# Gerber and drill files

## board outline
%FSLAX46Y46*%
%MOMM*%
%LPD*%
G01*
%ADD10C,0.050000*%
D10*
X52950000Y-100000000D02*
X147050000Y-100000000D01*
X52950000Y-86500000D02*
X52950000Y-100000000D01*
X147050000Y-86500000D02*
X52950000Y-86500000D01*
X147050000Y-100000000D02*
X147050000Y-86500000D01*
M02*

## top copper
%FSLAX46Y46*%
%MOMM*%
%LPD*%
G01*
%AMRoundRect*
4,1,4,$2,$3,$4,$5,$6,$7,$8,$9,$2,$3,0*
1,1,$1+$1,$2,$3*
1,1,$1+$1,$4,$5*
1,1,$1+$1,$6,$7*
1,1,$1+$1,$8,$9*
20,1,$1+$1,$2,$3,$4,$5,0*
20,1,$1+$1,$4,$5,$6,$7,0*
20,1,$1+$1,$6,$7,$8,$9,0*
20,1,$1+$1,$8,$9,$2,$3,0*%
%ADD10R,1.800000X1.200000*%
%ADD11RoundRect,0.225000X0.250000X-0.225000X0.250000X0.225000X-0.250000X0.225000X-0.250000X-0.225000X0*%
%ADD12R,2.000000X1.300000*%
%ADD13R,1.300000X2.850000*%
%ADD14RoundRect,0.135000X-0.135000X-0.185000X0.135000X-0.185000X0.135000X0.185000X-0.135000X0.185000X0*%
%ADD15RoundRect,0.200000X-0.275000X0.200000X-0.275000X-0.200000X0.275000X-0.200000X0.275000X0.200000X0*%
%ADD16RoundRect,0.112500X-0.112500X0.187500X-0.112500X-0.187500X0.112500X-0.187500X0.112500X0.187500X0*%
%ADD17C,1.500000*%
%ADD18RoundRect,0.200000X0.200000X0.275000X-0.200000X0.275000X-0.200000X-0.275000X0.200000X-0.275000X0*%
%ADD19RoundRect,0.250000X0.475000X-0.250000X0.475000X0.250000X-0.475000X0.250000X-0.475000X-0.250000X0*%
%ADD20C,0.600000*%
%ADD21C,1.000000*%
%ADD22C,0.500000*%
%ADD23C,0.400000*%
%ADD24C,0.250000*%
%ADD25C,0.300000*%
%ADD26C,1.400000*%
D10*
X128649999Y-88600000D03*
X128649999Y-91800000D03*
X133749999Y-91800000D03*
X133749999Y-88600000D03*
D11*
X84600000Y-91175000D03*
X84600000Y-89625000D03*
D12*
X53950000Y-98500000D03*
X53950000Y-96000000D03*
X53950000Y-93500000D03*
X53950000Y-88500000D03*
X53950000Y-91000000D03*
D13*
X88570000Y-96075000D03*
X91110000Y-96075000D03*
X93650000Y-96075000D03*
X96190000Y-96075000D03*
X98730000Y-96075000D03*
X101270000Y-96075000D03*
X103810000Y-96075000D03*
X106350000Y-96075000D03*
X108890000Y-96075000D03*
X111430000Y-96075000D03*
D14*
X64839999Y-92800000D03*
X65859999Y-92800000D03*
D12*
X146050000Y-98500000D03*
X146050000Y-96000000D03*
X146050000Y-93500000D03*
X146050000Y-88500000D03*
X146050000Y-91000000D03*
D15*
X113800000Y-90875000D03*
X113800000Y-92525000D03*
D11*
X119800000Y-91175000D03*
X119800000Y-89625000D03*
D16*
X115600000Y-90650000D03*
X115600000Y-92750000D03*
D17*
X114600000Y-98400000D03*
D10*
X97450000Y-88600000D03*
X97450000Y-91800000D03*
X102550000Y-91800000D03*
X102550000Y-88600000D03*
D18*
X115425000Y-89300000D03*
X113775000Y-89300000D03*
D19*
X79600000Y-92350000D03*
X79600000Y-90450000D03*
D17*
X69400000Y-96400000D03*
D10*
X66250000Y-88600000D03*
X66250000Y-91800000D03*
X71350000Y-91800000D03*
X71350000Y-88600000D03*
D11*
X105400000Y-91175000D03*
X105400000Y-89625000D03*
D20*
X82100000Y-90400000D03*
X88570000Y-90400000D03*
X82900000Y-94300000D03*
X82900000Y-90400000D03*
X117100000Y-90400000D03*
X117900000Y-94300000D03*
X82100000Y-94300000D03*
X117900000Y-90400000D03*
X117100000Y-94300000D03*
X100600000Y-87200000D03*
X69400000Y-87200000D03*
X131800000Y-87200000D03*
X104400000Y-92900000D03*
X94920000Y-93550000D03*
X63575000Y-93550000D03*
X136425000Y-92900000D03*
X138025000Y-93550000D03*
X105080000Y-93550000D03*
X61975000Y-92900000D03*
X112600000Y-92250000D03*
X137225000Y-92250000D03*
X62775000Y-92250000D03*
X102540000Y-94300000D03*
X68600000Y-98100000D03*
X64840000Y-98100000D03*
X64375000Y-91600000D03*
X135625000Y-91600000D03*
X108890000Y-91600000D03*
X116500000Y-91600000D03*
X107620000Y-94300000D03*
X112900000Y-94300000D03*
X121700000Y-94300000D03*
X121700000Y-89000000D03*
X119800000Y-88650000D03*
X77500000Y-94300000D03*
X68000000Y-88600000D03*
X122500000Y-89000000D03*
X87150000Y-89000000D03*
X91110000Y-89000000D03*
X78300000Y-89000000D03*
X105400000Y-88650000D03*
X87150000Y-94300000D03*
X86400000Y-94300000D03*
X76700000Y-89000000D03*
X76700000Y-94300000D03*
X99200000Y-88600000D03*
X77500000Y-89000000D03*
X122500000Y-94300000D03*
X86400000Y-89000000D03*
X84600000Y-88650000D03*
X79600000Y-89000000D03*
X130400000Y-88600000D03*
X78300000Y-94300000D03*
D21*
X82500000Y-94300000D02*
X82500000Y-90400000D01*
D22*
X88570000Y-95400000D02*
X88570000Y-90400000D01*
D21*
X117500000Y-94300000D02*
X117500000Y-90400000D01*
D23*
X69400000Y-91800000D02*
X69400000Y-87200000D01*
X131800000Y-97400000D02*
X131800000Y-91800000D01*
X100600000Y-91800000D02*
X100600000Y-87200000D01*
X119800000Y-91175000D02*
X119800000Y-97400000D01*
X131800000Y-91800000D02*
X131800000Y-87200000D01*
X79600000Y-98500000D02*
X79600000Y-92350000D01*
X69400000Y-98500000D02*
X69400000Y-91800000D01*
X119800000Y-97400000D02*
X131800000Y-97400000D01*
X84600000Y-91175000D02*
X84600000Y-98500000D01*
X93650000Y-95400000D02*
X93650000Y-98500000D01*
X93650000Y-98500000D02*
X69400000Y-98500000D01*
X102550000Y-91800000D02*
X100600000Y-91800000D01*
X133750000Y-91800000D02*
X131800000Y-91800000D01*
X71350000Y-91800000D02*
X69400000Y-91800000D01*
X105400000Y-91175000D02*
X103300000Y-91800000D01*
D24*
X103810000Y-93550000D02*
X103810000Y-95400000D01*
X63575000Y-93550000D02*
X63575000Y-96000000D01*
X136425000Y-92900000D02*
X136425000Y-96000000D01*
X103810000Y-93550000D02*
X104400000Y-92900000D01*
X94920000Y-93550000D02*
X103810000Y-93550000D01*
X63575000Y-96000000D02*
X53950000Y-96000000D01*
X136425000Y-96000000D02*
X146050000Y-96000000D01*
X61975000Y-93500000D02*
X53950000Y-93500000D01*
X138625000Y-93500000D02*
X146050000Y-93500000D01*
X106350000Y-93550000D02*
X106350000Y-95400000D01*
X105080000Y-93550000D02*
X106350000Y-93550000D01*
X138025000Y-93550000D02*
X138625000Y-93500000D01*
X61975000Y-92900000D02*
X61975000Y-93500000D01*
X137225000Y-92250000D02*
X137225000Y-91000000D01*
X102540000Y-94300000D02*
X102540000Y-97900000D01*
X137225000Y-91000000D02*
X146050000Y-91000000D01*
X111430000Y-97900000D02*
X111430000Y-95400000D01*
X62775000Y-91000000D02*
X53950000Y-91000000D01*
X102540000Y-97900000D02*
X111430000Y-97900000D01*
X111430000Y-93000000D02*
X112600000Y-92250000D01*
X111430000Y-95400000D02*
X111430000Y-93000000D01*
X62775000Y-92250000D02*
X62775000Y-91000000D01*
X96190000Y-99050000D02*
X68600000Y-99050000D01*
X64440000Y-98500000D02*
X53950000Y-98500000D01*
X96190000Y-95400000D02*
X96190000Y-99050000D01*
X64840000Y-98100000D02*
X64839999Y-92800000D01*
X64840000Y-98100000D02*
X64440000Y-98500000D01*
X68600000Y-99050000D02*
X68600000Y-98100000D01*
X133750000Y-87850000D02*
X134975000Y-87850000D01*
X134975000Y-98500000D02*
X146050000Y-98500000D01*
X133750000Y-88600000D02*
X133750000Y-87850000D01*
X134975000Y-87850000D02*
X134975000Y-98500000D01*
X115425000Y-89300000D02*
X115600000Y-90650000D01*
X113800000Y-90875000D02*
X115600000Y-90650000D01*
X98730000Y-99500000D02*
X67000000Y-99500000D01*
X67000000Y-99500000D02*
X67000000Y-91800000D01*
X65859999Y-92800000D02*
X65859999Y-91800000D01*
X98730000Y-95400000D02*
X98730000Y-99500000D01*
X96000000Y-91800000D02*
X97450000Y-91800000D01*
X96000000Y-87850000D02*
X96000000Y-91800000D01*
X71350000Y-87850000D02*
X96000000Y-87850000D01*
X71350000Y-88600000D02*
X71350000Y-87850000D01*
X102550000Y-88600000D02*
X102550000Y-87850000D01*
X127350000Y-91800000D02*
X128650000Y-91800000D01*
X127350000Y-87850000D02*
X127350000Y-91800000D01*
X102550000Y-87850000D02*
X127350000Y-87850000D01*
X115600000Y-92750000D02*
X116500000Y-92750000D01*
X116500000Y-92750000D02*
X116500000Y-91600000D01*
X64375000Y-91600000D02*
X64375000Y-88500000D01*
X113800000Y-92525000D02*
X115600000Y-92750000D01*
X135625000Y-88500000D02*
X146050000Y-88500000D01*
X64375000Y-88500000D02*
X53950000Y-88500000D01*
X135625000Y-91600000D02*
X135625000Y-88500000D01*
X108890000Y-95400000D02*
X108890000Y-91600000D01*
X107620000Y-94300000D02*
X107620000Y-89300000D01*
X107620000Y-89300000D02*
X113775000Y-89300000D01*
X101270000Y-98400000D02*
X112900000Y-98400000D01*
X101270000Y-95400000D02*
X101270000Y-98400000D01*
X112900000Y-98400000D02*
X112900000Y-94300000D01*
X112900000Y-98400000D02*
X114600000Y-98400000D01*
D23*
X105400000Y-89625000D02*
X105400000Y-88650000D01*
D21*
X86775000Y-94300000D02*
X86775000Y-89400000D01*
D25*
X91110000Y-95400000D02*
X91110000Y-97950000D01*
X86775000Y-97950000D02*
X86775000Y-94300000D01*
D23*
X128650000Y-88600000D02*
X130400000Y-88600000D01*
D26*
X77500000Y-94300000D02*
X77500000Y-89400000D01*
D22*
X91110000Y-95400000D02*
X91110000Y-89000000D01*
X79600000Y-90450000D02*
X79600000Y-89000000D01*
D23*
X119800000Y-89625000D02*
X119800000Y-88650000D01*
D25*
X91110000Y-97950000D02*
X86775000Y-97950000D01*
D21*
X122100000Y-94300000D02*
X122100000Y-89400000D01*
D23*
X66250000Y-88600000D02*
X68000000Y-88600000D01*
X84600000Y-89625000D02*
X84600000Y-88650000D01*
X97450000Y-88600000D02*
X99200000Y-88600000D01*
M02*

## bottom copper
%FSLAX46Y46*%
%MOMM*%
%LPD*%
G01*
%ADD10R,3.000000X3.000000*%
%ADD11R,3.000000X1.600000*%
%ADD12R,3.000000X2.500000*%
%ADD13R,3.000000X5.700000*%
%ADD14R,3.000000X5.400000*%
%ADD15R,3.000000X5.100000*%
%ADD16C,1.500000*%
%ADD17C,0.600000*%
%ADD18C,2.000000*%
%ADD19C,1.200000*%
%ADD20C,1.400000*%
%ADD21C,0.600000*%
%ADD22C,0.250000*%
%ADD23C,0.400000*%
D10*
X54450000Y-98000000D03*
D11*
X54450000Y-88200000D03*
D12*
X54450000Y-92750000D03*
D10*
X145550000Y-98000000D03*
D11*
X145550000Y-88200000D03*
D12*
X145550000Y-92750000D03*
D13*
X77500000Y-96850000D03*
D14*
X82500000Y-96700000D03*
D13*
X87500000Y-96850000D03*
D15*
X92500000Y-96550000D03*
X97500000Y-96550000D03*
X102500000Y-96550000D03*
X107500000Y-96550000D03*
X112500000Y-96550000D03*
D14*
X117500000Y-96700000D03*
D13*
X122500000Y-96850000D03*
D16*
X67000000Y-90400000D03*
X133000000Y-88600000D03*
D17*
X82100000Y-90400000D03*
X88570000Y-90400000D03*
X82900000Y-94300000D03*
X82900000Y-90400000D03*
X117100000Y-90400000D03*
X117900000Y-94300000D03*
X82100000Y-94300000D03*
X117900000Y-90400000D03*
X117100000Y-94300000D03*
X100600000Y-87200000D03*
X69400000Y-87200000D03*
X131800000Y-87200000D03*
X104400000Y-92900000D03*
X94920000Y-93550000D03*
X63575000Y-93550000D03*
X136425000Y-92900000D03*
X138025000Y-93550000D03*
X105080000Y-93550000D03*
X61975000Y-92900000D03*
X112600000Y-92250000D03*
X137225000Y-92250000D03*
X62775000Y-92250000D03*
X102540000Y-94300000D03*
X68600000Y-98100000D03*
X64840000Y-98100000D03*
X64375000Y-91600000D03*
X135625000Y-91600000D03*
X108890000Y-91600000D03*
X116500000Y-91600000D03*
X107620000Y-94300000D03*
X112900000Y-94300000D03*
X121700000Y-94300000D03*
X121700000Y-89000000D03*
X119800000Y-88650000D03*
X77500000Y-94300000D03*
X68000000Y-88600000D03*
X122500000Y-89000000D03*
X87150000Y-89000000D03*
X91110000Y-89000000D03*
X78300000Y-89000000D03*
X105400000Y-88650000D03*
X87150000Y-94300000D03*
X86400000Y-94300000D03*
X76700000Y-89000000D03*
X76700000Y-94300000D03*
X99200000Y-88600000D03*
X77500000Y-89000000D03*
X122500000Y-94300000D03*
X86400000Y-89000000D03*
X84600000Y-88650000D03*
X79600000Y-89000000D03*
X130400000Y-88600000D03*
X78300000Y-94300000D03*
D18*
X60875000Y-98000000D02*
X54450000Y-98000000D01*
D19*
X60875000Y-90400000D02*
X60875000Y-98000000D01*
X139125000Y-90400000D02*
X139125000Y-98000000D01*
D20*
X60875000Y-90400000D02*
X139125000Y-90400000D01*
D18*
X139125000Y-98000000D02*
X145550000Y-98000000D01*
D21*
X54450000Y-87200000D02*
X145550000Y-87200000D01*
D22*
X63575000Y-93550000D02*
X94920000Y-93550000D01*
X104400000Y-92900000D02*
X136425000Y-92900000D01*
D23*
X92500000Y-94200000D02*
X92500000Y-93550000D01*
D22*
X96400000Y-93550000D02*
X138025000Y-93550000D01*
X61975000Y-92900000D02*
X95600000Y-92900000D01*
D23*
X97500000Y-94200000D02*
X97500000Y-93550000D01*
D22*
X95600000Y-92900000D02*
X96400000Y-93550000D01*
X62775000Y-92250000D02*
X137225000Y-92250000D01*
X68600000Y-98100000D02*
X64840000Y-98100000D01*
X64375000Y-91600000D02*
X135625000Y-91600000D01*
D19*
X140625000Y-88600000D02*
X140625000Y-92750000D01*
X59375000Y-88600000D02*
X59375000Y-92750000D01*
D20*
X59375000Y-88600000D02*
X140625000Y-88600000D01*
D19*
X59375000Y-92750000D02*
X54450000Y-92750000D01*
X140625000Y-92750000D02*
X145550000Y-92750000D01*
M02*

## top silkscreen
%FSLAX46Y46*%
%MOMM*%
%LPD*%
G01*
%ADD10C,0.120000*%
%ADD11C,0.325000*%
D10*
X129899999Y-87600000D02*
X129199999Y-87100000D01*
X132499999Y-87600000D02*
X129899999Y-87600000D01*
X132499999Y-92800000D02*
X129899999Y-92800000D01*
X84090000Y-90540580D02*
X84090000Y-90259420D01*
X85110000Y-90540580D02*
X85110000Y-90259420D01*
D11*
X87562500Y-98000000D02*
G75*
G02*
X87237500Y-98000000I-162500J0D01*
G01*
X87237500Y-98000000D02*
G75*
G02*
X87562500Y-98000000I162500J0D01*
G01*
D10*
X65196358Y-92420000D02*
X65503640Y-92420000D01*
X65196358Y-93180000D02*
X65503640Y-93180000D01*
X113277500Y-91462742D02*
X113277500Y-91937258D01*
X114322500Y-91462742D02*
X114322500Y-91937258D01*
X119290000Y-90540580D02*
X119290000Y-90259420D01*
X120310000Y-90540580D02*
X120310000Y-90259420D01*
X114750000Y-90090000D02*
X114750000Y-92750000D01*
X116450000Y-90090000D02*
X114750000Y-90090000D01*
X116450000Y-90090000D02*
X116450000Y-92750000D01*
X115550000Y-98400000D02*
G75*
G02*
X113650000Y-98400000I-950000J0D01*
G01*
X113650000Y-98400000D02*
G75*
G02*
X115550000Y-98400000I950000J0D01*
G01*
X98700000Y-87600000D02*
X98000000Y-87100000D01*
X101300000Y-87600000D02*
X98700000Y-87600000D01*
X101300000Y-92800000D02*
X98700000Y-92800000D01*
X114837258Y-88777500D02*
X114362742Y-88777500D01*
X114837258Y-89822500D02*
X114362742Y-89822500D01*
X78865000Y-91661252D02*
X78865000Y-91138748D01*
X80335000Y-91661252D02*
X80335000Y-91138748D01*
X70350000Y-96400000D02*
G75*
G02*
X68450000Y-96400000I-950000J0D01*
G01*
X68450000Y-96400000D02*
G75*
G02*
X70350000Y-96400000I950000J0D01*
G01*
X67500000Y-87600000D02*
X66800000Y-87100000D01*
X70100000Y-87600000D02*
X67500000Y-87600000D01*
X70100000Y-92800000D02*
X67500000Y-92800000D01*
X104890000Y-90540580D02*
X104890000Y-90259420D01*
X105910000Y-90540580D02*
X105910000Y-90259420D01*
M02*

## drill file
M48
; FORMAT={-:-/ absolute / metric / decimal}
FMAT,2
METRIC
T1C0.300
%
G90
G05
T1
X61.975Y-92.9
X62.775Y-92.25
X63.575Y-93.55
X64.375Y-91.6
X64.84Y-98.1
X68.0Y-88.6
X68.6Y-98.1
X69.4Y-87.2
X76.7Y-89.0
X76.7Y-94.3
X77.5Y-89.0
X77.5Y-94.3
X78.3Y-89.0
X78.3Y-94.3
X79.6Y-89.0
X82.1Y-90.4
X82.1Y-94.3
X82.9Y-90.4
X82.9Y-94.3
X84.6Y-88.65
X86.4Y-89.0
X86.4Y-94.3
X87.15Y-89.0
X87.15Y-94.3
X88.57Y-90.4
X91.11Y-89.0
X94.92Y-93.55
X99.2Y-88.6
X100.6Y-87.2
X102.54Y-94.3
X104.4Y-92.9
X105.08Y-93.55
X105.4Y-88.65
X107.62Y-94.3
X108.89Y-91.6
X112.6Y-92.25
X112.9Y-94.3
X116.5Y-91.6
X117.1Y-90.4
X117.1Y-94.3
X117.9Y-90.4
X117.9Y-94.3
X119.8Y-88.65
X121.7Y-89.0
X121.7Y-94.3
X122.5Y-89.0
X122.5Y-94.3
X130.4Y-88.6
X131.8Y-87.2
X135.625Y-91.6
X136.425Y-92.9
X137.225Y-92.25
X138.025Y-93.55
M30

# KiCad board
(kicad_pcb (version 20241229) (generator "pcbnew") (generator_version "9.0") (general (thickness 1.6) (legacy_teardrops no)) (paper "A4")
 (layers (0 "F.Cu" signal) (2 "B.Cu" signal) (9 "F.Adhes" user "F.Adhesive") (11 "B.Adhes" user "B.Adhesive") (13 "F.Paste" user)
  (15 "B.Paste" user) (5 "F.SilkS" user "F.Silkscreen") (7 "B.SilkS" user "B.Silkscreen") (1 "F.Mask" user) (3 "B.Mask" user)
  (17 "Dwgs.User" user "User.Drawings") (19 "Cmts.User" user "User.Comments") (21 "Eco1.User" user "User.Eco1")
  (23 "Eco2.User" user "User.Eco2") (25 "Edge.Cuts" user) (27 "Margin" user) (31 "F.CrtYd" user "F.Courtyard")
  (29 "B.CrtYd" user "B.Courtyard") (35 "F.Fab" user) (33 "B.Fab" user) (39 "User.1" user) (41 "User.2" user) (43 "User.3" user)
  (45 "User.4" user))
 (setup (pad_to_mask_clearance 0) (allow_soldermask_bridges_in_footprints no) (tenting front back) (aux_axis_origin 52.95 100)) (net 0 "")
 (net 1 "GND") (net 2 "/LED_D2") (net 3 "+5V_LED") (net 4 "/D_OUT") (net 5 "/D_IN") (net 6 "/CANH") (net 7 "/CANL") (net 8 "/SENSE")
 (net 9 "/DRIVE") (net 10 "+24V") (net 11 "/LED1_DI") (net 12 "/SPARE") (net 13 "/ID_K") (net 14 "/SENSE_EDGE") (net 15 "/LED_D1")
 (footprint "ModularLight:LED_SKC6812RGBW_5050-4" (layer "F.Cu") (at 131.199999 90.2 180)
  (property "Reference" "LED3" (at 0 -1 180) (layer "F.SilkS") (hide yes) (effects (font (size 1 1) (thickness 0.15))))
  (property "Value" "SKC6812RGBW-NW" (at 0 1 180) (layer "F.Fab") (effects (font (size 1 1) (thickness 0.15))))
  (fp_line (start 1.3 2.6) (end 2 3.1) (stroke (width 0.12) (type solid)) (layer "F.SilkS"))
  (fp_line (start -1.3 2.6) (end 1.3 2.6) (stroke (width 0.12) (type solid)) (layer "F.SilkS"))
  (fp_line (start -1.3 -2.6) (end 1.3 -2.6) (stroke (width 0.12) (type solid)) (layer "F.SilkS"))
  (pad "1" smd rect (at 2.55 1.6 180) (size 1.8 1.2) (layers "F.Cu" "F.Mask" "F.Paste") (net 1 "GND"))
  (pad "2" smd rect (at 2.55 -1.6 180) (size 1.8 1.2) (layers "F.Cu" "F.Mask" "F.Paste") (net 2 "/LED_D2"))
  (pad "3" smd rect (at -2.55 -1.6 180) (size 1.8 1.2) (layers "F.Cu" "F.Mask" "F.Paste") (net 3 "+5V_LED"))
  (pad "4" smd rect (at -2.55 1.6 180) (size 1.8 1.2) (layers "F.Cu" "F.Mask" "F.Paste") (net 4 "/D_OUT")))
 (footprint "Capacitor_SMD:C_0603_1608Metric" (layer "F.Cu") (at 84.6 90.4 90)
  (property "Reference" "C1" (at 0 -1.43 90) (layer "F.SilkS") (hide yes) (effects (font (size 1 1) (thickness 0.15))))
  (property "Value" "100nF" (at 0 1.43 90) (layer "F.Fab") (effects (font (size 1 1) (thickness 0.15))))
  (fp_line (start -0.14058 -0.51) (end 0.14058 -0.51) (stroke (width 0.12) (type solid)) (layer "F.SilkS"))
  (fp_line (start -0.14058 0.51) (end 0.14058 0.51) (stroke (width 0.12) (type solid)) (layer "F.SilkS"))
  (pad "1" smd roundrect (at -0.775 0 90) (size 0.9 0.95) (layers "F.Cu" "F.Mask" "F.Paste") (roundrect_rratio 0.25) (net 3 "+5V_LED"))
  (pad "2" smd roundrect (at 0.775 0 90) (size 0.9 0.95) (layers "F.Cu" "F.Mask" "F.Paste") (roundrect_rratio 0.25) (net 1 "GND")))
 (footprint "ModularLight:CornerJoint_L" (layer "F.Cu") (at 52.95 100)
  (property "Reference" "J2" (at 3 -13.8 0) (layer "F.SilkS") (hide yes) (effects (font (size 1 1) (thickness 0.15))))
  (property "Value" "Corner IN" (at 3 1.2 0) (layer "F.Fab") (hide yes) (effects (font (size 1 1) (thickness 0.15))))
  (pad "1" smd rect (at 1 -1.5) (size 2 1.3) (layers "F.Cu" "F.Mask" "F.Paste") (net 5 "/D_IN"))
  (pad "2" smd rect (at 1 -4) (size 2 1.3) (layers "F.Cu" "F.Mask" "F.Paste") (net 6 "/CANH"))
  (pad "3" smd rect (at 1 -6.5) (size 2 1.3) (layers "F.Cu" "F.Mask" "F.Paste") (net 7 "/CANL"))
  (pad "4" smd rect (at 1 -11.5) (size 2 1.3) (layers "F.Cu" "F.Mask" "F.Paste") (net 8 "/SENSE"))
  (pad "5" smd rect (at 1 -9) (size 2 1.3) (layers "F.Cu" "F.Mask" "F.Paste") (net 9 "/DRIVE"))
  (pad "6" smd rect (at 1.5 -2) (size 3 3) (layers "B.Cu" "B.Mask") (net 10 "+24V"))
  (pad "7" smd rect (at 1.5 -11.8) (size 3 1.6) (layers "B.Cu" "B.Mask") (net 3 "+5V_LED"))
  (pad "8" smd rect (at 1.5 -7.25) (size 3 2.5) (layers "B.Cu" "B.Mask") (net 1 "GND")))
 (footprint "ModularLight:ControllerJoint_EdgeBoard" (layer "F.Cu") (at 100 94.75)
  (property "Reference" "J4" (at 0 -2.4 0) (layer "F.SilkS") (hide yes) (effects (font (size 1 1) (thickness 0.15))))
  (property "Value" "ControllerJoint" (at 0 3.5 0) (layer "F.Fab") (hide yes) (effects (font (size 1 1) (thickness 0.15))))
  (fp_circle (center -12.6 3.25) (end -12.35 3.25) (stroke (width 0.15) (type solid)) (fill yes) (layer "F.SilkS"))
  (pad "1" smd rect (at -11.43 1.325) (size 1.3 2.85) (layers "F.Cu" "F.Mask" "F.Paste") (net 10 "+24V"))
  (pad "2" smd rect (at -8.89 1.325) (size 1.3 2.85) (layers "F.Cu" "F.Mask" "F.Paste") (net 1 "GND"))
  (pad "3" smd rect (at -6.35 1.325) (size 1.3 2.85) (layers "F.Cu" "F.Mask" "F.Paste") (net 3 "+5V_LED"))
  (pad "4" smd rect (at -3.81 1.325) (size 1.3 2.85) (layers "F.Cu" "F.Mask" "F.Paste") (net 5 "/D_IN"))
  (pad "5" smd rect (at -1.27 1.325) (size 1.3 2.85) (layers "F.Cu" "F.Mask" "F.Paste") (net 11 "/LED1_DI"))
  (pad "6" smd rect (at 1.27 1.325) (size 1.3 2.85) (layers "F.Cu" "F.Mask" "F.Paste") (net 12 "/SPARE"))
  (pad "7" smd rect (at 3.81 1.325) (size 1.3 2.85) (layers "F.Cu" "F.Mask" "F.Paste") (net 6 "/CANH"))
  (pad "8" smd rect (at 6.35 1.325) (size 1.3 2.85) (layers "F.Cu" "F.Mask" "F.Paste") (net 7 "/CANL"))
  (pad "9" smd rect (at 8.89 1.325) (size 1.3 2.85) (layers "F.Cu" "F.Mask" "F.Paste") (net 8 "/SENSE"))
  (pad "10" smd rect (at 11.43 1.325) (size 1.3 2.85) (layers "F.Cu" "F.Mask" "F.Paste") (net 9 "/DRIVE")))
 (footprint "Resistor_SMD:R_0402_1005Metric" (layer "F.Cu") (at 65.349999 92.8)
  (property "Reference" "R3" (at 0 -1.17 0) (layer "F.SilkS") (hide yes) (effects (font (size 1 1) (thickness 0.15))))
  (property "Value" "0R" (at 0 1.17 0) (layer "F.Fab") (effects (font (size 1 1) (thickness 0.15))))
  (fp_line (start -0.153641 -0.38) (end 0.153641 -0.38) (stroke (width 0.12) (type solid)) (layer "F.SilkS"))
  (fp_line (start -0.153641 0.38) (end 0.153641 0.38) (stroke (width 0.12) (type solid)) (layer "F.SilkS"))
  (pad "1" smd roundrect (at -0.51 0) (size 0.54 0.64) (layers "F.Cu" "F.Mask" "F.Paste") (roundrect_rratio 0.25) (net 5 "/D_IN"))
  (pad "2" smd roundrect (at 0.51 0) (size 0.54 0.64) (layers "F.Cu" "F.Mask" "F.Paste") (roundrect_rratio 0.25) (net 11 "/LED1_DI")))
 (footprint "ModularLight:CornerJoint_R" (layer "F.Cu") (at 147.05 100)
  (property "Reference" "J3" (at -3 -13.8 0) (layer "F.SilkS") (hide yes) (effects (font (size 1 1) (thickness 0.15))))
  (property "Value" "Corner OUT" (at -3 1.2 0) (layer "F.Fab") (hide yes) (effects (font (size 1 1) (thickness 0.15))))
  (pad "1" smd rect (at -1 -1.5) (size 2 1.3) (layers "F.Cu" "F.Mask" "F.Paste") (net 4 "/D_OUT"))
  (pad "2" smd rect (at -1 -4) (size 2 1.3) (layers "F.Cu" "F.Mask" "F.Paste") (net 6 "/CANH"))
  (pad "3" smd rect (at -1 -6.5) (size 2 1.3) (layers "F.Cu" "F.Mask" "F.Paste") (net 7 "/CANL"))
  (pad "4" smd rect (at -1 -11.5) (size 2 1.3) (layers "F.Cu" "F.Mask" "F.Paste") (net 8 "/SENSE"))
  (pad "5" smd rect (at -1 -9) (size 2 1.3) (layers "F.Cu" "F.Mask" "F.Paste") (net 9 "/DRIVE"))
  (pad "6" smd rect (at -1.5 -2) (size 3 3) (layers "B.Cu" "B.Mask") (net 10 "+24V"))
  (pad "7" smd rect (at -1.5 -11.8) (size 3 1.6) (layers "B.Cu" "B.Mask") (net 3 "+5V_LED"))
  (pad "8" smd rect (at -1.5 -7.25) (size 3 2.5) (layers "B.Cu" "B.Mask") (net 1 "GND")))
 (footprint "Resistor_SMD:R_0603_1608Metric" (layer "F.Cu") (at 113.8 91.7 -90)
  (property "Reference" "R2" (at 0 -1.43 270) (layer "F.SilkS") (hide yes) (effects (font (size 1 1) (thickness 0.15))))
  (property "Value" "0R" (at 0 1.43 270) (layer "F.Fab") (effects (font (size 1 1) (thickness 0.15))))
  (fp_line (start -0.237258 0.5225) (end 0.237258 0.5225) (stroke (width 0.12) (type solid)) (layer "F.SilkS"))
  (fp_line (start -0.237258 -0.5225) (end 0.237258 -0.5225) (stroke (width 0.12) (type solid)) (layer "F.SilkS"))
  (pad "1" smd roundrect (at -0.825 0 270) (size 0.8 0.95) (layers "F.Cu" "F.Mask" "F.Paste") (roundrect_rratio 0.25) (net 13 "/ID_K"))
  (pad "2" smd roundrect (at 0.825 0 270) (size 0.8 0.95) (layers "F.Cu" "F.Mask" "F.Paste") (roundrect_rratio 0.25) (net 8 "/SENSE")))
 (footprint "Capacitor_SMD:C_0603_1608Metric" (layer "F.Cu") (at 119.8 90.4 90)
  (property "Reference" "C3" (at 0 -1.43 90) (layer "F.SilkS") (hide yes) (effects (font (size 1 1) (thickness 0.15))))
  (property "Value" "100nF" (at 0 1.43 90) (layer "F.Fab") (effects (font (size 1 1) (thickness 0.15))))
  (fp_line (start -0.14058 -0.51) (end 0.14058 -0.51) (stroke (width 0.12) (type solid)) (layer "F.SilkS"))
  (fp_line (start -0.14058 0.51) (end 0.14058 0.51) (stroke (width 0.12) (type solid)) (layer "F.SilkS"))
  (pad "1" smd roundrect (at -0.775 0 90) (size 0.9 0.95) (layers "F.Cu" "F.Mask" "F.Paste") (roundrect_rratio 0.25) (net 3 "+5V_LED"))
  (pad "2" smd roundrect (at 0.775 0 90) (size 0.9 0.95) (layers "F.Cu" "F.Mask" "F.Paste") (roundrect_rratio 0.25) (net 1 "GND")))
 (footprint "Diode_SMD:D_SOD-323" (layer "F.Cu") (at 115.6 91.7 -90)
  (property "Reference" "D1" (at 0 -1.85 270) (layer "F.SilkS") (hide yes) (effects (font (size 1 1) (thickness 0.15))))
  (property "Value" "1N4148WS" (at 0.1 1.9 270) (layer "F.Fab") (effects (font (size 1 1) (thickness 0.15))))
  (fp_line (start -1.61 0.85) (end 1.05 0.85) (stroke (width 0.12) (type solid)) (layer "F.SilkS"))
  (fp_line (start -1.61 -0.85) (end -1.61 0.85) (stroke (width 0.12) (type solid)) (layer "F.SilkS"))
  (fp_line (start -1.61 -0.85) (end 1.05 -0.85) (stroke (width 0.12) (type solid)) (layer "F.SilkS"))
  (pad "1" smd roundrect (at -1.05 0 270) (size 0.6 0.45) (layers "F.Cu" "F.Mask" "F.Paste") (roundrect_rratio 0.25) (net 13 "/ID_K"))
  (pad "2" smd roundrect (at 1.05 0 270) (size 0.6 0.45) (layers "F.Cu" "F.Mask" "F.Paste") (roundrect_rratio 0.25) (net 8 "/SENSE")))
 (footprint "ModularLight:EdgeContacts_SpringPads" (layer "F.Cu") (at 100 100)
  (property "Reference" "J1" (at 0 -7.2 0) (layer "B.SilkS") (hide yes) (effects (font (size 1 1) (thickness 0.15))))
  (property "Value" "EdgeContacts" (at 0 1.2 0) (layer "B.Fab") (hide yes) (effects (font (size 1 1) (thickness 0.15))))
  (pad "X1" smd rect (at -22.5 -3.15) (size 3 5.7) (layers "B.Cu" "B.Mask") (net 1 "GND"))
  (pad "X2" smd rect (at -17.5 -3.3) (size 3 5.4) (layers "B.Cu" "B.Mask") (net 10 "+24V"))
  (pad "X3" smd rect (at -12.5 -3.15) (size 3 5.7) (layers "B.Cu" "B.Mask") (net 1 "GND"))
  (pad "X4" smd rect (at -7.5 -3.45) (size 3 5.1) (layers "B.Cu" "B.Mask") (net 6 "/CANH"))
  (pad "X5" smd rect (at -2.5 -3.45) (size 3 5.1) (layers "B.Cu" "B.Mask") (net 7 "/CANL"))
  (pad "X6" smd rect (at 2.5 -3.45) (size 3 5.1) (layers "B.Cu" "B.Mask") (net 9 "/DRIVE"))
  (pad "X7" smd rect (at 7.5 -3.45) (size 3 5.1) (layers "B.Cu" "B.Mask") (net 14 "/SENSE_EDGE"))
  (pad "X8" smd rect (at 12.5 -3.45) (size 3 5.1) (layers "B.Cu" "B.Mask") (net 12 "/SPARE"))
  (pad "X9" smd rect (at 17.5 -3.3) (size 3 5.4) (layers "B.Cu" "B.Mask") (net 10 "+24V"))
  (pad "X10" smd rect (at 22.5 -3.15) (size 3 5.7) (layers "B.Cu" "B.Mask") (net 1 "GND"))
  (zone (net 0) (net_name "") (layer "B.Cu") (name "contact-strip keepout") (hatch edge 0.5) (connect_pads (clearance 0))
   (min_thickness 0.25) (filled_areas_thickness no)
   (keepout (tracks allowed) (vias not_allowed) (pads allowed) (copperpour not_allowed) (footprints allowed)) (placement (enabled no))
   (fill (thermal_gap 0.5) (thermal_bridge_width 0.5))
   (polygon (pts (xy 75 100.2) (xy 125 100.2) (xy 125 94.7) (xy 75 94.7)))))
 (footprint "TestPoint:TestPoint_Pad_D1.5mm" (layer "F.Cu") (at 114.6 98.4)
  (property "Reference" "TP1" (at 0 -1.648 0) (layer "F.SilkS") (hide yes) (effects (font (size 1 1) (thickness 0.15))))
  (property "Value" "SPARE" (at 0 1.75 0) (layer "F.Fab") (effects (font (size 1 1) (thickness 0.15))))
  (fp_circle (center 0 0) (end 0 0.95) (stroke (width 0.12) (type solid)) (fill no) (layer "F.SilkS"))
  (pad "1" smd circle (at 0 0) (size 1.5 1.5) (layers "F.Cu" "F.Mask") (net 12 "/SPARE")))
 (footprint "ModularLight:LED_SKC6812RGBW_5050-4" (layer "F.Cu") (at 100 90.2 180)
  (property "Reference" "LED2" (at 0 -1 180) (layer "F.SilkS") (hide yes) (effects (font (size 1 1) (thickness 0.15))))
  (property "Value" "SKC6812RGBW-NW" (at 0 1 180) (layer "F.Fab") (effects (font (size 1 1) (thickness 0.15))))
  (fp_line (start 1.3 2.6) (end 2 3.1) (stroke (width 0.12) (type solid)) (layer "F.SilkS"))
  (fp_line (start -1.3 2.6) (end 1.3 2.6) (stroke (width 0.12) (type solid)) (layer "F.SilkS"))
  (fp_line (start -1.3 -2.6) (end 1.3 -2.6) (stroke (width 0.12) (type solid)) (layer "F.SilkS"))
  (pad "1" smd rect (at 2.55 1.6 180) (size 1.8 1.2) (layers "F.Cu" "F.Mask" "F.Paste") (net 1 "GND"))
  (pad "2" smd rect (at 2.55 -1.6 180) (size 1.8 1.2) (layers "F.Cu" "F.Mask" "F.Paste") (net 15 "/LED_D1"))
  (pad "3" smd rect (at -2.55 -1.6 180) (size 1.8 1.2) (layers "F.Cu" "F.Mask" "F.Paste") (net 3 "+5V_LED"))
  (pad "4" smd rect (at -2.55 1.6 180) (size 1.8 1.2) (layers "F.Cu" "F.Mask" "F.Paste") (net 2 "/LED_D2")))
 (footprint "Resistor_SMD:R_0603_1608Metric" (layer "F.Cu") (at 114.6 89.3 180)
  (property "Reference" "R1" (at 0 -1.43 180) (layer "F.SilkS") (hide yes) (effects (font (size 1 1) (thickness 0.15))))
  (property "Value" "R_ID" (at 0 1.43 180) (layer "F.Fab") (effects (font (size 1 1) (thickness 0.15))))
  (fp_line (start -0.237258 0.5225) (end 0.237258 0.5225) (stroke (width 0.12) (type solid)) (layer "F.SilkS"))
  (fp_line (start -0.237258 -0.5225) (end 0.237258 -0.5225) (stroke (width 0.12) (type solid)) (layer "F.SilkS"))
  (pad "1" smd roundrect (at -0.825 0 180) (size 0.8 0.95) (layers "F.Cu" "F.Mask" "F.Paste") (roundrect_rratio 0.25) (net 13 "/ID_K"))
  (pad "2" smd roundrect (at 0.825 0 180) (size 0.8 0.95) (layers "F.Cu" "F.Mask" "F.Paste") (roundrect_rratio 0.25) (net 14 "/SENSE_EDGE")))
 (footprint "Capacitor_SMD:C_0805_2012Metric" (layer "F.Cu") (at 79.6 91.4 90)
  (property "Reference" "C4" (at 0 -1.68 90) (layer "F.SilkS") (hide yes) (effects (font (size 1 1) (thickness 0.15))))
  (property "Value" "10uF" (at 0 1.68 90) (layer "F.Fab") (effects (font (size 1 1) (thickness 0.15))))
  (fp_line (start -0.261252 -0.735) (end 0.261252 -0.735) (stroke (width 0.12) (type solid)) (layer "F.SilkS"))
  (fp_line (start -0.261252 0.735) (end 0.261252 0.735) (stroke (width 0.12) (type solid)) (layer "F.SilkS"))
  (pad "1" smd roundrect (at -0.95 0 90) (size 1 1.45) (layers "F.Cu" "F.Mask" "F.Paste") (roundrect_rratio 0.25) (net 3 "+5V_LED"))
  (pad "2" smd roundrect (at 0.95 0 90) (size 1 1.45) (layers "F.Cu" "F.Mask" "F.Paste") (roundrect_rratio 0.25) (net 1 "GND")))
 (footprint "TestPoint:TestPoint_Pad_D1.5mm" (layer "F.Cu") (at 69.4 96.4)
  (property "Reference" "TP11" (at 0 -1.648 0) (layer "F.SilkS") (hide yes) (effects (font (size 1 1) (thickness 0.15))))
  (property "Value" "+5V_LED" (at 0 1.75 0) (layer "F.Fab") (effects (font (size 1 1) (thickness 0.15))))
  (fp_circle (center 0 0) (end 0 0.95) (stroke (width 0.12) (type solid)) (fill no) (layer "F.SilkS"))
  (pad "1" smd circle (at 0 0) (size 1.5 1.5) (layers "F.Cu" "F.Mask") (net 3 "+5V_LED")))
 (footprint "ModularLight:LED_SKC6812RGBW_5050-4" (layer "F.Cu") (at 68.8 90.2 180)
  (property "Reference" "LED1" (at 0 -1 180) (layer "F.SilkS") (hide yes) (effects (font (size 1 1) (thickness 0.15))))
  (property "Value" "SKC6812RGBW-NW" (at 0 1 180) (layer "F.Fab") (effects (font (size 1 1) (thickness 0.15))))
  (fp_line (start 1.3 2.6) (end 2 3.1) (stroke (width 0.12) (type solid)) (layer "F.SilkS"))
  (fp_line (start -1.3 2.6) (end 1.3 2.6) (stroke (width 0.12) (type solid)) (layer "F.SilkS"))
  (fp_line (start -1.3 -2.6) (end 1.3 -2.6) (stroke (width 0.12) (type solid)) (layer "F.SilkS"))
  (pad "1" smd rect (at 2.55 1.6 180) (size 1.8 1.2) (layers "F.Cu" "F.Mask" "F.Paste") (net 1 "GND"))
  (pad "2" smd rect (at 2.55 -1.6 180) (size 1.8 1.2) (layers "F.Cu" "F.Mask" "F.Paste") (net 11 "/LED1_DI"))
  (pad "3" smd rect (at -2.55 -1.6 180) (size 1.8 1.2) (layers "F.Cu" "F.Mask" "F.Paste") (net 3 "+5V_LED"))
  (pad "4" smd rect (at -2.55 1.6 180) (size 1.8 1.2) (layers "F.Cu" "F.Mask" "F.Paste") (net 15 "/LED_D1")))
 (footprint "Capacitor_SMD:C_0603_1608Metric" (layer "F.Cu") (at 105.4 90.4 90)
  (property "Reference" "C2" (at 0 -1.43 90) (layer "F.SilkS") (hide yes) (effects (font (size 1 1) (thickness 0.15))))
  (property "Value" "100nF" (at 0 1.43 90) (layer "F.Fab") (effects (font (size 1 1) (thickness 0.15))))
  (fp_line (start -0.14058 -0.51) (end 0.14058 -0.51) (stroke (width 0.12) (type solid)) (layer "F.SilkS"))
  (fp_line (start -0.14058 0.51) (end 0.14058 0.51) (stroke (width 0.12) (type solid)) (layer "F.SilkS"))
  (pad "1" smd roundrect (at -0.775 0 90) (size 0.9 0.95) (layers "F.Cu" "F.Mask" "F.Paste") (roundrect_rratio 0.25) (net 3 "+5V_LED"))
  (pad "2" smd roundrect (at 0.775 0 90) (size 0.9 0.95) (layers "F.Cu" "F.Mask" "F.Paste") (roundrect_rratio 0.25) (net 1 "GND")))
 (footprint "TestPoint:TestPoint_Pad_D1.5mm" (layer "B.Cu") (at 67 90.4 180)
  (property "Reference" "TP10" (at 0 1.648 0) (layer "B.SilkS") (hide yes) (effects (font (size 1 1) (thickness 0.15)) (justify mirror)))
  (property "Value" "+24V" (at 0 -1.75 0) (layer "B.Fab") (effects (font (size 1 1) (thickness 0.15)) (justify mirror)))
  (pad "1" smd circle (at 0 0 180) (size 1.5 1.5) (layers "B.Cu" "B.Mask") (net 10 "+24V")))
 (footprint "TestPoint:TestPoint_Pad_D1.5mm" (layer "B.Cu") (at 133 88.6 180)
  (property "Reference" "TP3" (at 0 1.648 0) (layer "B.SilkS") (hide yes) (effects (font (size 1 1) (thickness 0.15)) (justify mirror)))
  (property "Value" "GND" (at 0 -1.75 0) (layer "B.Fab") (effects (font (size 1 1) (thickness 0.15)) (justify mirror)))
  (pad "1" smd circle (at 0 0 180) (size 1.5 1.5) (layers "B.Cu" "B.Mask") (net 1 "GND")))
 (gr_line (start 52.95 100) (end 147.05 100) (stroke (width 0.05) (type default)) (layer "Edge.Cuts"))
 (gr_line (start 52.95 86.5) (end 52.95 100) (stroke (width 0.05) (type default)) (layer "Edge.Cuts"))
 (gr_line (start 147.05 86.5) (end 52.95 86.5) (stroke (width 0.05) (type default)) (layer "Edge.Cuts"))
 (gr_line (start 147.05 100) (end 147.05 86.5) (stroke (width 0.05) (type default)) (layer "Edge.Cuts"))
 (segment (start 82.5 94.3) (end 82.5 90.4) (width 1) (locked yes) (layer "F.Cu") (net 10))
 (segment (start 88.57 95.4) (end 88.57 90.4) (width 0.5) (locked yes) (layer "F.Cu") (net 10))
 (segment (start 117.5 94.3) (end 117.5 90.4) (width 1) (locked yes) (layer "F.Cu") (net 10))
 (via (at 82.1 90.4) (size 0.6) (drill 0.3) (layers "F.Cu" "B.Cu") (locked yes) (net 10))
 (via (at 88.57 90.4) (size 0.6) (drill 0.3) (layers "F.Cu" "B.Cu") (locked yes) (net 10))
 (via (at 82.9 94.3) (size 0.6) (drill 0.3) (layers "F.Cu" "B.Cu") (locked yes) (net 10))
 (via (at 82.9 90.4) (size 0.6) (drill 0.3) (layers "F.Cu" "B.Cu") (locked yes) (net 10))
 (via (at 117.1 90.4) (size 0.6) (drill 0.3) (layers "F.Cu" "B.Cu") (locked yes) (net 10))
 (via (at 117.9 94.3) (size 0.6) (drill 0.3) (layers "F.Cu" "B.Cu") (locked yes) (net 10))
 (via (at 82.1 94.3) (size 0.6) (drill 0.3) (layers "F.Cu" "B.Cu") (locked yes) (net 10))
 (via (at 117.9 90.4) (size 0.6) (drill 0.3) (layers "F.Cu" "B.Cu") (locked yes) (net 10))
 (via (at 117.1 94.3) (size 0.6) (drill 0.3) (layers "F.Cu" "B.Cu") (locked yes) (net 10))
 (segment (start 60.875 98) (end 54.45 98) (width 2) (locked yes) (layer "B.Cu") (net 10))
 (segment (start 60.875 90.4) (end 60.875 98) (width 1.2) (locked yes) (layer "B.Cu") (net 10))
 (segment (start 139.125 90.4) (end 139.125 98) (width 1.2) (locked yes) (layer "B.Cu") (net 10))
 (segment (start 60.875 90.4) (end 139.125 90.4) (width 1.4) (locked yes) (layer "B.Cu") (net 10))
 (segment (start 139.125 98) (end 145.55 98) (width 2) (locked yes) (layer "B.Cu") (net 10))
 (segment (start 69.4 91.8) (end 69.4 87.2) (width 0.4) (locked yes) (layer "F.Cu") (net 3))
 (segment (start 131.8 97.4) (end 131.8 91.8) (width 0.4) (locked yes) (layer "F.Cu") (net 3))
 (segment (start 100.6 91.8) (end 100.6 87.2) (width 0.4) (locked yes) (layer "F.Cu") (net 3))
 (segment (start 119.8 91.175) (end 119.8 97.4) (width 0.4) (locked yes) (layer "F.Cu") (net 3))
 (segment (start 131.8 91.8) (end 131.8 87.2) (width 0.4) (locked yes) (layer "F.Cu") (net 3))
 (segment (start 79.6 98.5) (end 79.6 92.35) (width 0.4) (locked yes) (layer "F.Cu") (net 3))
 (segment (start 69.4 98.5) (end 69.4 91.8) (width 0.4) (locked yes) (layer "F.Cu") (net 3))
 (segment (start 119.8 97.4) (end 131.8 97.4) (width 0.4) (locked yes) (layer "F.Cu") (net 3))
 (segment (start 84.6 91.175) (end 84.6 98.5) (width 0.4) (locked yes) (layer "F.Cu") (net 3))
 (segment (start 93.65 95.4) (end 93.65 98.5) (width 0.4) (locked yes) (layer "F.Cu") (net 3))
 (segment (start 93.65 98.5) (end 69.4 98.5) (width 0.4) (locked yes) (layer "F.Cu") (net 3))
 (segment (start 102.55 91.8) (end 100.6 91.8) (width 0.4) (locked yes) (layer "F.Cu") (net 3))
 (segment (start 133.75 91.8) (end 131.8 91.8) (width 0.4) (locked yes) (layer "F.Cu") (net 3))
 (segment (start 71.35 91.8) (end 69.4 91.8) (width 0.4) (locked yes) (layer "F.Cu") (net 3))
 (segment (start 105.4 91.175) (end 103.3 91.8) (width 0.4) (locked yes) (layer "F.Cu") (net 3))
 (via (at 100.6 87.2) (size 0.6) (drill 0.3) (layers "F.Cu" "B.Cu") (locked yes) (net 3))
 (via (at 69.4 87.2) (size 0.6) (drill 0.3) (layers "F.Cu" "B.Cu") (locked yes) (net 3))
 (via (at 131.8 87.2) (size 0.6) (drill 0.3) (layers "F.Cu" "B.Cu") (locked yes) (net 3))
 (segment (start 54.45 87.2) (end 145.55 87.2) (width 0.6) (locked yes) (layer "B.Cu") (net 3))
 (segment (start 103.81 93.55) (end 103.81 95.4) (width 0.25) (locked yes) (layer "F.Cu") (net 6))
 (segment (start 63.575 93.55) (end 63.575 96) (width 0.25) (locked yes) (layer "F.Cu") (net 6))
 (segment (start 136.425 92.9) (end 136.425 96) (width 0.25) (locked yes) (layer "F.Cu") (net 6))
 (segment (start 103.81 93.55) (end 104.4 92.9) (width 0.25) (locked yes) (layer "F.Cu") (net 6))
 (segment (start 94.92 93.55) (end 103.81 93.55) (width 0.25) (locked yes) (layer "F.Cu") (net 6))
 (segment (start 63.575 96) (end 53.95 96) (width 0.25) (locked yes) (layer "F.Cu") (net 6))
 (segment (start 136.425 96) (end 146.05 96) (width 0.25) (locked yes) (layer "F.Cu") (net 6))
 (via (at 104.4 92.9) (size 0.6) (drill 0.3) (layers "F.Cu" "B.Cu") (locked yes) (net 6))
 (via (at 94.92 93.55) (size 0.6) (drill 0.3) (layers "F.Cu" "B.Cu") (locked yes) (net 6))
 (via (at 63.575 93.55) (size 0.6) (drill 0.3) (layers "F.Cu" "B.Cu") (locked yes) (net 6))
 (via (at 136.425 92.9) (size 0.6) (drill 0.3) (layers "F.Cu" "B.Cu") (locked yes) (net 6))
 (segment (start 63.575 93.55) (end 94.92 93.55) (width 0.25) (locked yes) (layer "B.Cu") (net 6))
 (segment (start 104.4 92.9) (end 136.425 92.9) (width 0.25) (locked yes) (layer "B.Cu") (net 6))
 (segment (start 92.5 94.2) (end 92.5 93.55) (width 0.4) (locked yes) (layer "B.Cu") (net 6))
 (segment (start 61.975 93.5) (end 53.95 93.5) (width 0.25) (locked yes) (layer "F.Cu") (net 7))
 (segment (start 138.625 93.5) (end 146.05 93.5) (width 0.25) (locked yes) (layer "F.Cu") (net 7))
 (segment (start 106.35 93.55) (end 106.35 95.4) (width 0.25) (locked yes) (layer "F.Cu") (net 7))
 (segment (start 105.08 93.55) (end 106.35 93.55) (width 0.25) (locked yes) (layer "F.Cu") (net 7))
 (segment (start 138.025 93.55) (end 138.625 93.5) (width 0.25) (locked yes) (layer "F.Cu") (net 7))
 (segment (start 61.975 92.9) (end 61.975 93.5) (width 0.25) (locked yes) (layer "F.Cu") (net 7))
 (via (at 138.025 93.55) (size 0.6) (drill 0.3) (layers "F.Cu" "B.Cu") (locked yes) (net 7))
 (via (at 105.08 93.55) (size 0.6) (drill 0.3) (layers "F.Cu" "B.Cu") (locked yes) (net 7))
 (via (at 61.975 92.9) (size 0.6) (drill 0.3) (layers "F.Cu" "B.Cu") (locked yes) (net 7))
 (segment (start 96.4 93.55) (end 138.025 93.55) (width 0.25) (locked yes) (layer "B.Cu") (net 7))
 (segment (start 61.975 92.9) (end 95.6 92.9) (width 0.25) (locked yes) (layer "B.Cu") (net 7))
 (segment (start 97.5 94.2) (end 97.5 93.55) (width 0.4) (locked yes) (layer "B.Cu") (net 7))
 (segment (start 95.6 92.9) (end 96.4 93.55) (width 0.25) (locked yes) (layer "B.Cu") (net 7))
 (segment (start 137.225 92.25) (end 137.225 91) (width 0.25) (locked yes) (layer "F.Cu") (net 9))
 (segment (start 102.54 94.3) (end 102.54 97.9) (width 0.25) (locked yes) (layer "F.Cu") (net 9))
 (segment (start 137.225 91) (end 146.05 91) (width 0.25) (locked yes) (layer "F.Cu") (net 9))
 (segment (start 111.43 97.9) (end 111.43 95.4) (width 0.25) (locked yes) (layer "F.Cu") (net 9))
 (segment (start 62.775 91) (end 53.95 91) (width 0.25) (locked yes) (layer "F.Cu") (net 9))
 (segment (start 102.54 97.9) (end 111.43 97.9) (width 0.25) (locked yes) (layer "F.Cu") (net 9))
 (segment (start 111.43 93) (end 112.6 92.25) (width 0.25) (locked yes) (layer "F.Cu") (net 9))
 (segment (start 111.43 95.4) (end 111.43 93) (width 0.25) (locked yes) (layer "F.Cu") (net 9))
 (segment (start 62.775 92.25) (end 62.775 91) (width 0.25) (locked yes) (layer "F.Cu") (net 9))
 (via (at 112.6 92.25) (size 0.6) (drill 0.3) (layers "F.Cu" "B.Cu") (locked yes) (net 9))
 (via (at 137.225 92.25) (size 0.6) (drill 0.3) (layers "F.Cu" "B.Cu") (locked yes) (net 9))
 (via (at 62.775 92.25) (size 0.6) (drill 0.3) (layers "F.Cu" "B.Cu") (locked yes) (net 9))
 (via (at 102.54 94.3) (size 0.6) (drill 0.3) (layers "F.Cu" "B.Cu") (locked yes) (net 9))
 (segment (start 62.775 92.25) (end 137.225 92.25) (width 0.25) (locked yes) (layer "B.Cu") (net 9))
 (segment (start 96.19 99.05) (end 68.6 99.05) (width 0.25) (locked yes) (layer "F.Cu") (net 5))
 (segment (start 64.44 98.5) (end 53.95 98.5) (width 0.25) (locked yes) (layer "F.Cu") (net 5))
 (segment (start 96.19 95.4) (end 96.19 99.05) (width 0.25) (locked yes) (layer "F.Cu") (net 5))
 (segment (start 64.84 98.1) (end 64.839999 92.8) (width 0.25) (locked yes) (layer "F.Cu") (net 5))
 (segment (start 64.84 98.1) (end 64.44 98.5) (width 0.25) (locked yes) (layer "F.Cu") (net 5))
 (segment (start 68.6 99.05) (end 68.6 98.1) (width 0.25) (locked yes) (layer "F.Cu") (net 5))
 (via (at 68.6 98.1) (size 0.6) (drill 0.3) (layers "F.Cu" "B.Cu") (locked yes) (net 5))
 (via (at 64.84 98.1) (size 0.6) (drill 0.3) (layers "F.Cu" "B.Cu") (locked yes) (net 5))
 (segment (start 68.6 98.1) (end 64.84 98.1) (width 0.25) (locked yes) (layer "B.Cu") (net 5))
 (segment (start 133.75 87.85) (end 134.975 87.85) (width 0.25) (locked yes) (layer "F.Cu") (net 4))
 (segment (start 134.975 98.5) (end 146.05 98.5) (width 0.25) (locked yes) (layer "F.Cu") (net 4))
 (segment (start 133.75 88.6) (end 133.75 87.85) (width 0.25) (locked yes) (layer "F.Cu") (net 4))
 (segment (start 134.975 87.85) (end 134.975 98.5) (width 0.25) (locked yes) (layer "F.Cu") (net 4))
 (segment (start 115.425 89.3) (end 115.6 90.65) (width 0.25) (locked yes) (layer "F.Cu") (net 13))
 (segment (start 113.8 90.875) (end 115.6 90.65) (width 0.25) (locked yes) (layer "F.Cu") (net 13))
 (segment (start 98.73 99.5) (end 67 99.5) (width 0.25) (locked yes) (layer "F.Cu") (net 11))
 (segment (start 67 99.5) (end 67 91.8) (width 0.25) (locked yes) (layer "F.Cu") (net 11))
 (segment (start 65.859999 92.8) (end 65.859999 91.8) (width 0.25) (locked yes) (layer "F.Cu") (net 11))
 (segment (start 98.73 95.4) (end 98.73 99.5) (width 0.25) (locked yes) (layer "F.Cu") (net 11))
 (segment (start 96 91.8) (end 97.45 91.8) (width 0.25) (locked yes) (layer "F.Cu") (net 15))
 (segment (start 96 87.85) (end 96 91.8) (width 0.25) (locked yes) (layer "F.Cu") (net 15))
 (segment (start 71.35 87.85) (end 96 87.85) (width 0.25) (locked yes) (layer "F.Cu") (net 15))
 (segment (start 71.35 88.6) (end 71.35 87.85) (width 0.25) (locked yes) (layer "F.Cu") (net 15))
 (segment (start 102.55 88.6) (end 102.55 87.85) (width 0.25) (locked yes) (layer "F.Cu") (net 2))
 (segment (start 127.35 91.8) (end 128.65 91.8) (width 0.25) (locked yes) (layer "F.Cu") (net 2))
 (segment (start 127.35 87.85) (end 127.35 91.8) (width 0.25) (locked yes) (layer "F.Cu") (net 2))
 (segment (start 102.55 87.85) (end 127.35 87.85) (width 0.25) (locked yes) (layer "F.Cu") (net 2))
 (segment (start 115.6 92.75) (end 116.5 92.75) (width 0.25) (locked yes) (layer "F.Cu") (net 8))
 (segment (start 116.5 92.75) (end 116.5 91.6) (width 0.25) (locked yes) (layer "F.Cu") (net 8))
 (segment (start 64.375 91.6) (end 64.375 88.5) (width 0.25) (locked yes) (layer "F.Cu") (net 8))
 (segment (start 113.8 92.525) (end 115.6 92.75) (width 0.25) (locked yes) (layer "F.Cu") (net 8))
 (segment (start 135.625 88.5) (end 146.05 88.5) (width 0.25) (locked yes) (layer "F.Cu") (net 8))
 (segment (start 64.375 88.5) (end 53.95 88.5) (width 0.25) (locked yes) (layer "F.Cu") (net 8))
 (segment (start 135.625 91.6) (end 135.625 88.5) (width 0.25) (locked yes) (layer "F.Cu") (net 8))
 (segment (start 108.89 95.4) (end 108.89 91.6) (width 0.25) (locked yes) (layer "F.Cu") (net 8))
 (via (at 64.375 91.6) (size 0.6) (drill 0.3) (layers "F.Cu" "B.Cu") (locked yes) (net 8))
 (via (at 135.625 91.6) (size 0.6) (drill 0.3) (layers "F.Cu" "B.Cu") (locked yes) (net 8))
 (via (at 108.89 91.6) (size 0.6) (drill 0.3) (layers "F.Cu" "B.Cu") (locked yes) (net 8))
 (via (at 116.5 91.6) (size 0.6) (drill 0.3) (layers "F.Cu" "B.Cu") (locked yes) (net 8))
 (segment (start 64.375 91.6) (end 135.625 91.6) (width 0.25) (locked yes) (layer "B.Cu") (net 8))
 (segment (start 107.62 94.3) (end 107.62 89.3) (width 0.25) (locked yes) (layer "F.Cu") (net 14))
 (segment (start 107.62 89.3) (end 113.775 89.3) (width 0.25) (locked yes) (layer "F.Cu") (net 14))
 (via (at 107.62 94.3) (size 0.6) (drill 0.3) (layers "F.Cu" "B.Cu") (locked yes) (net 14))
 (segment (start 101.27 98.4) (end 112.9 98.4) (width 0.25) (locked yes) (layer "F.Cu") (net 12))
 (segment (start 101.27 95.4) (end 101.27 98.4) (width 0.25) (locked yes) (layer "F.Cu") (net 12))
 (segment (start 112.9 98.4) (end 112.9 94.3) (width 0.25) (locked yes) (layer "F.Cu") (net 12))
 (segment (start 112.9 98.4) (end 114.6 98.4) (width 0.25) (locked yes) (layer "F.Cu") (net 12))
 (via (at 112.9 94.3) (size 0.6) (drill 0.3) (layers "F.Cu" "B.Cu") (locked yes) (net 12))
 (segment (start 105.4 89.625) (end 105.4 88.65) (width 0.4) (locked yes) (layer "F.Cu") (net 1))
 (segment (start 86.775 94.3) (end 86.775 89.4) (width 1) (locked yes) (layer "F.Cu") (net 1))
 (segment (start 91.11 95.4) (end 91.11 97.95) (width 0.3) (locked yes) (layer "F.Cu") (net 1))
 (segment (start 86.775 97.95) (end 86.775 94.3) (width 0.3) (locked yes) (layer "F.Cu") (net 1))
 (segment (start 128.65 88.6) (end 130.4 88.6) (width 0.4) (locked yes) (layer "F.Cu") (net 1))
 (segment (start 77.5 94.3) (end 77.5 89.4) (width 1.4) (locked yes) (layer "F.Cu") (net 1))
 (segment (start 91.11 95.4) (end 91.11 89) (width 0.5) (locked yes) (layer "F.Cu") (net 1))
 (segment (start 79.6 90.45) (end 79.6 89) (width 0.5) (locked yes) (layer "F.Cu") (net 1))
 (segment (start 119.8 89.625) (end 119.8 88.65) (width 0.4) (locked yes) (layer "F.Cu") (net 1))
 (segment (start 91.11 97.95) (end 86.775 97.95) (width 0.3) (locked yes) (layer "F.Cu") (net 1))
 (segment (start 122.1 94.3) (end 122.1 89.4) (width 1) (locked yes) (layer "F.Cu") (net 1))
 (segment (start 66.25 88.6) (end 68 88.6) (width 0.4) (locked yes) (layer "F.Cu") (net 1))
 (segment (start 84.6 89.625) (end 84.6 88.65) (width 0.4) (locked yes) (layer "F.Cu") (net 1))
 (segment (start 97.45 88.6) (end 99.2 88.6) (width 0.4) (locked yes) (layer "F.Cu") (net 1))
 (via (at 121.7 94.3) (size 0.6) (drill 0.3) (layers "F.Cu" "B.Cu") (locked yes) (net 1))
 (via (at 121.7 89) (size 0.6) (drill 0.3) (layers "F.Cu" "B.Cu") (locked yes) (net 1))
 (via (at 119.8 88.65) (size 0.6) (drill 0.3) (layers "F.Cu" "B.Cu") (locked yes) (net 1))
 (via (at 77.5 94.3) (size 0.6) (drill 0.3) (layers "F.Cu" "B.Cu") (locked yes) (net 1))
 (via (at 68 88.6) (size 0.6) (drill 0.3) (layers "F.Cu" "B.Cu") (locked yes) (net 1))
 (via (at 122.5 89) (size 0.6) (drill 0.3) (layers "F.Cu" "B.Cu") (locked yes) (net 1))
 (via (at 87.15 89) (size 0.6) (drill 0.3) (layers "F.Cu" "B.Cu") (locked yes) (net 1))
 (via (at 91.11 89) (size 0.6) (drill 0.3) (layers "F.Cu" "B.Cu") (locked yes) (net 1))
 (via (at 78.3 89) (size 0.6) (drill 0.3) (layers "F.Cu" "B.Cu") (locked yes) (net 1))
 (via (at 105.4 88.65) (size 0.6) (drill 0.3) (layers "F.Cu" "B.Cu") (locked yes) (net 1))
 (via (at 87.15 94.3) (size 0.6) (drill 0.3) (layers "F.Cu" "B.Cu") (locked yes) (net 1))
 (via (at 86.4 94.3) (size 0.6) (drill 0.3) (layers "F.Cu" "B.Cu") (locked yes) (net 1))
 (via (at 76.7 89) (size 0.6) (drill 0.3) (layers "F.Cu" "B.Cu") (locked yes) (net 1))
 (via (at 76.7 94.3) (size 0.6) (drill 0.3) (layers "F.Cu" "B.Cu") (locked yes) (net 1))
 (via (at 99.2 88.6) (size 0.6) (drill 0.3) (layers "F.Cu" "B.Cu") (locked yes) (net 1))
 (via (at 77.5 89) (size 0.6) (drill 0.3) (layers "F.Cu" "B.Cu") (locked yes) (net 1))
 (via (at 122.5 94.3) (size 0.6) (drill 0.3) (layers "F.Cu" "B.Cu") (locked yes) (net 1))
 (via (at 86.4 89) (size 0.6) (drill 0.3) (layers "F.Cu" "B.Cu") (locked yes) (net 1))
 (via (at 84.6 88.65) (size 0.6) (drill 0.3) (layers "F.Cu" "B.Cu") (locked yes) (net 1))
 (via (at 79.6 89) (size 0.6) (drill 0.3) (layers "F.Cu" "B.Cu") (locked yes) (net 1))
 (via (at 130.4 88.6) (size 0.6) (drill 0.3) (layers "F.Cu" "B.Cu") (locked yes) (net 1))
 (via (at 78.3 94.3) (size 0.6) (drill 0.3) (layers "F.Cu" "B.Cu") (locked yes) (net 1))
 (segment (start 140.625 88.6) (end 140.625 92.75) (width 1.2) (locked yes) (layer "B.Cu") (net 1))
 (segment (start 59.375 88.6) (end 59.375 92.75) (width 1.2) (locked yes) (layer "B.Cu") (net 1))
 (segment (start 59.375 88.6) (end 140.625 88.6) (width 1.4) (locked yes) (layer "B.Cu") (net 1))
 (segment (start 59.375 92.75) (end 54.45 92.75) (width 1.2) (locked yes) (layer "B.Cu") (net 1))
 (segment (start 140.625 92.75) (end 145.55 92.75) (width 1.2) (locked yes) (layer "B.Cu") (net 1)))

